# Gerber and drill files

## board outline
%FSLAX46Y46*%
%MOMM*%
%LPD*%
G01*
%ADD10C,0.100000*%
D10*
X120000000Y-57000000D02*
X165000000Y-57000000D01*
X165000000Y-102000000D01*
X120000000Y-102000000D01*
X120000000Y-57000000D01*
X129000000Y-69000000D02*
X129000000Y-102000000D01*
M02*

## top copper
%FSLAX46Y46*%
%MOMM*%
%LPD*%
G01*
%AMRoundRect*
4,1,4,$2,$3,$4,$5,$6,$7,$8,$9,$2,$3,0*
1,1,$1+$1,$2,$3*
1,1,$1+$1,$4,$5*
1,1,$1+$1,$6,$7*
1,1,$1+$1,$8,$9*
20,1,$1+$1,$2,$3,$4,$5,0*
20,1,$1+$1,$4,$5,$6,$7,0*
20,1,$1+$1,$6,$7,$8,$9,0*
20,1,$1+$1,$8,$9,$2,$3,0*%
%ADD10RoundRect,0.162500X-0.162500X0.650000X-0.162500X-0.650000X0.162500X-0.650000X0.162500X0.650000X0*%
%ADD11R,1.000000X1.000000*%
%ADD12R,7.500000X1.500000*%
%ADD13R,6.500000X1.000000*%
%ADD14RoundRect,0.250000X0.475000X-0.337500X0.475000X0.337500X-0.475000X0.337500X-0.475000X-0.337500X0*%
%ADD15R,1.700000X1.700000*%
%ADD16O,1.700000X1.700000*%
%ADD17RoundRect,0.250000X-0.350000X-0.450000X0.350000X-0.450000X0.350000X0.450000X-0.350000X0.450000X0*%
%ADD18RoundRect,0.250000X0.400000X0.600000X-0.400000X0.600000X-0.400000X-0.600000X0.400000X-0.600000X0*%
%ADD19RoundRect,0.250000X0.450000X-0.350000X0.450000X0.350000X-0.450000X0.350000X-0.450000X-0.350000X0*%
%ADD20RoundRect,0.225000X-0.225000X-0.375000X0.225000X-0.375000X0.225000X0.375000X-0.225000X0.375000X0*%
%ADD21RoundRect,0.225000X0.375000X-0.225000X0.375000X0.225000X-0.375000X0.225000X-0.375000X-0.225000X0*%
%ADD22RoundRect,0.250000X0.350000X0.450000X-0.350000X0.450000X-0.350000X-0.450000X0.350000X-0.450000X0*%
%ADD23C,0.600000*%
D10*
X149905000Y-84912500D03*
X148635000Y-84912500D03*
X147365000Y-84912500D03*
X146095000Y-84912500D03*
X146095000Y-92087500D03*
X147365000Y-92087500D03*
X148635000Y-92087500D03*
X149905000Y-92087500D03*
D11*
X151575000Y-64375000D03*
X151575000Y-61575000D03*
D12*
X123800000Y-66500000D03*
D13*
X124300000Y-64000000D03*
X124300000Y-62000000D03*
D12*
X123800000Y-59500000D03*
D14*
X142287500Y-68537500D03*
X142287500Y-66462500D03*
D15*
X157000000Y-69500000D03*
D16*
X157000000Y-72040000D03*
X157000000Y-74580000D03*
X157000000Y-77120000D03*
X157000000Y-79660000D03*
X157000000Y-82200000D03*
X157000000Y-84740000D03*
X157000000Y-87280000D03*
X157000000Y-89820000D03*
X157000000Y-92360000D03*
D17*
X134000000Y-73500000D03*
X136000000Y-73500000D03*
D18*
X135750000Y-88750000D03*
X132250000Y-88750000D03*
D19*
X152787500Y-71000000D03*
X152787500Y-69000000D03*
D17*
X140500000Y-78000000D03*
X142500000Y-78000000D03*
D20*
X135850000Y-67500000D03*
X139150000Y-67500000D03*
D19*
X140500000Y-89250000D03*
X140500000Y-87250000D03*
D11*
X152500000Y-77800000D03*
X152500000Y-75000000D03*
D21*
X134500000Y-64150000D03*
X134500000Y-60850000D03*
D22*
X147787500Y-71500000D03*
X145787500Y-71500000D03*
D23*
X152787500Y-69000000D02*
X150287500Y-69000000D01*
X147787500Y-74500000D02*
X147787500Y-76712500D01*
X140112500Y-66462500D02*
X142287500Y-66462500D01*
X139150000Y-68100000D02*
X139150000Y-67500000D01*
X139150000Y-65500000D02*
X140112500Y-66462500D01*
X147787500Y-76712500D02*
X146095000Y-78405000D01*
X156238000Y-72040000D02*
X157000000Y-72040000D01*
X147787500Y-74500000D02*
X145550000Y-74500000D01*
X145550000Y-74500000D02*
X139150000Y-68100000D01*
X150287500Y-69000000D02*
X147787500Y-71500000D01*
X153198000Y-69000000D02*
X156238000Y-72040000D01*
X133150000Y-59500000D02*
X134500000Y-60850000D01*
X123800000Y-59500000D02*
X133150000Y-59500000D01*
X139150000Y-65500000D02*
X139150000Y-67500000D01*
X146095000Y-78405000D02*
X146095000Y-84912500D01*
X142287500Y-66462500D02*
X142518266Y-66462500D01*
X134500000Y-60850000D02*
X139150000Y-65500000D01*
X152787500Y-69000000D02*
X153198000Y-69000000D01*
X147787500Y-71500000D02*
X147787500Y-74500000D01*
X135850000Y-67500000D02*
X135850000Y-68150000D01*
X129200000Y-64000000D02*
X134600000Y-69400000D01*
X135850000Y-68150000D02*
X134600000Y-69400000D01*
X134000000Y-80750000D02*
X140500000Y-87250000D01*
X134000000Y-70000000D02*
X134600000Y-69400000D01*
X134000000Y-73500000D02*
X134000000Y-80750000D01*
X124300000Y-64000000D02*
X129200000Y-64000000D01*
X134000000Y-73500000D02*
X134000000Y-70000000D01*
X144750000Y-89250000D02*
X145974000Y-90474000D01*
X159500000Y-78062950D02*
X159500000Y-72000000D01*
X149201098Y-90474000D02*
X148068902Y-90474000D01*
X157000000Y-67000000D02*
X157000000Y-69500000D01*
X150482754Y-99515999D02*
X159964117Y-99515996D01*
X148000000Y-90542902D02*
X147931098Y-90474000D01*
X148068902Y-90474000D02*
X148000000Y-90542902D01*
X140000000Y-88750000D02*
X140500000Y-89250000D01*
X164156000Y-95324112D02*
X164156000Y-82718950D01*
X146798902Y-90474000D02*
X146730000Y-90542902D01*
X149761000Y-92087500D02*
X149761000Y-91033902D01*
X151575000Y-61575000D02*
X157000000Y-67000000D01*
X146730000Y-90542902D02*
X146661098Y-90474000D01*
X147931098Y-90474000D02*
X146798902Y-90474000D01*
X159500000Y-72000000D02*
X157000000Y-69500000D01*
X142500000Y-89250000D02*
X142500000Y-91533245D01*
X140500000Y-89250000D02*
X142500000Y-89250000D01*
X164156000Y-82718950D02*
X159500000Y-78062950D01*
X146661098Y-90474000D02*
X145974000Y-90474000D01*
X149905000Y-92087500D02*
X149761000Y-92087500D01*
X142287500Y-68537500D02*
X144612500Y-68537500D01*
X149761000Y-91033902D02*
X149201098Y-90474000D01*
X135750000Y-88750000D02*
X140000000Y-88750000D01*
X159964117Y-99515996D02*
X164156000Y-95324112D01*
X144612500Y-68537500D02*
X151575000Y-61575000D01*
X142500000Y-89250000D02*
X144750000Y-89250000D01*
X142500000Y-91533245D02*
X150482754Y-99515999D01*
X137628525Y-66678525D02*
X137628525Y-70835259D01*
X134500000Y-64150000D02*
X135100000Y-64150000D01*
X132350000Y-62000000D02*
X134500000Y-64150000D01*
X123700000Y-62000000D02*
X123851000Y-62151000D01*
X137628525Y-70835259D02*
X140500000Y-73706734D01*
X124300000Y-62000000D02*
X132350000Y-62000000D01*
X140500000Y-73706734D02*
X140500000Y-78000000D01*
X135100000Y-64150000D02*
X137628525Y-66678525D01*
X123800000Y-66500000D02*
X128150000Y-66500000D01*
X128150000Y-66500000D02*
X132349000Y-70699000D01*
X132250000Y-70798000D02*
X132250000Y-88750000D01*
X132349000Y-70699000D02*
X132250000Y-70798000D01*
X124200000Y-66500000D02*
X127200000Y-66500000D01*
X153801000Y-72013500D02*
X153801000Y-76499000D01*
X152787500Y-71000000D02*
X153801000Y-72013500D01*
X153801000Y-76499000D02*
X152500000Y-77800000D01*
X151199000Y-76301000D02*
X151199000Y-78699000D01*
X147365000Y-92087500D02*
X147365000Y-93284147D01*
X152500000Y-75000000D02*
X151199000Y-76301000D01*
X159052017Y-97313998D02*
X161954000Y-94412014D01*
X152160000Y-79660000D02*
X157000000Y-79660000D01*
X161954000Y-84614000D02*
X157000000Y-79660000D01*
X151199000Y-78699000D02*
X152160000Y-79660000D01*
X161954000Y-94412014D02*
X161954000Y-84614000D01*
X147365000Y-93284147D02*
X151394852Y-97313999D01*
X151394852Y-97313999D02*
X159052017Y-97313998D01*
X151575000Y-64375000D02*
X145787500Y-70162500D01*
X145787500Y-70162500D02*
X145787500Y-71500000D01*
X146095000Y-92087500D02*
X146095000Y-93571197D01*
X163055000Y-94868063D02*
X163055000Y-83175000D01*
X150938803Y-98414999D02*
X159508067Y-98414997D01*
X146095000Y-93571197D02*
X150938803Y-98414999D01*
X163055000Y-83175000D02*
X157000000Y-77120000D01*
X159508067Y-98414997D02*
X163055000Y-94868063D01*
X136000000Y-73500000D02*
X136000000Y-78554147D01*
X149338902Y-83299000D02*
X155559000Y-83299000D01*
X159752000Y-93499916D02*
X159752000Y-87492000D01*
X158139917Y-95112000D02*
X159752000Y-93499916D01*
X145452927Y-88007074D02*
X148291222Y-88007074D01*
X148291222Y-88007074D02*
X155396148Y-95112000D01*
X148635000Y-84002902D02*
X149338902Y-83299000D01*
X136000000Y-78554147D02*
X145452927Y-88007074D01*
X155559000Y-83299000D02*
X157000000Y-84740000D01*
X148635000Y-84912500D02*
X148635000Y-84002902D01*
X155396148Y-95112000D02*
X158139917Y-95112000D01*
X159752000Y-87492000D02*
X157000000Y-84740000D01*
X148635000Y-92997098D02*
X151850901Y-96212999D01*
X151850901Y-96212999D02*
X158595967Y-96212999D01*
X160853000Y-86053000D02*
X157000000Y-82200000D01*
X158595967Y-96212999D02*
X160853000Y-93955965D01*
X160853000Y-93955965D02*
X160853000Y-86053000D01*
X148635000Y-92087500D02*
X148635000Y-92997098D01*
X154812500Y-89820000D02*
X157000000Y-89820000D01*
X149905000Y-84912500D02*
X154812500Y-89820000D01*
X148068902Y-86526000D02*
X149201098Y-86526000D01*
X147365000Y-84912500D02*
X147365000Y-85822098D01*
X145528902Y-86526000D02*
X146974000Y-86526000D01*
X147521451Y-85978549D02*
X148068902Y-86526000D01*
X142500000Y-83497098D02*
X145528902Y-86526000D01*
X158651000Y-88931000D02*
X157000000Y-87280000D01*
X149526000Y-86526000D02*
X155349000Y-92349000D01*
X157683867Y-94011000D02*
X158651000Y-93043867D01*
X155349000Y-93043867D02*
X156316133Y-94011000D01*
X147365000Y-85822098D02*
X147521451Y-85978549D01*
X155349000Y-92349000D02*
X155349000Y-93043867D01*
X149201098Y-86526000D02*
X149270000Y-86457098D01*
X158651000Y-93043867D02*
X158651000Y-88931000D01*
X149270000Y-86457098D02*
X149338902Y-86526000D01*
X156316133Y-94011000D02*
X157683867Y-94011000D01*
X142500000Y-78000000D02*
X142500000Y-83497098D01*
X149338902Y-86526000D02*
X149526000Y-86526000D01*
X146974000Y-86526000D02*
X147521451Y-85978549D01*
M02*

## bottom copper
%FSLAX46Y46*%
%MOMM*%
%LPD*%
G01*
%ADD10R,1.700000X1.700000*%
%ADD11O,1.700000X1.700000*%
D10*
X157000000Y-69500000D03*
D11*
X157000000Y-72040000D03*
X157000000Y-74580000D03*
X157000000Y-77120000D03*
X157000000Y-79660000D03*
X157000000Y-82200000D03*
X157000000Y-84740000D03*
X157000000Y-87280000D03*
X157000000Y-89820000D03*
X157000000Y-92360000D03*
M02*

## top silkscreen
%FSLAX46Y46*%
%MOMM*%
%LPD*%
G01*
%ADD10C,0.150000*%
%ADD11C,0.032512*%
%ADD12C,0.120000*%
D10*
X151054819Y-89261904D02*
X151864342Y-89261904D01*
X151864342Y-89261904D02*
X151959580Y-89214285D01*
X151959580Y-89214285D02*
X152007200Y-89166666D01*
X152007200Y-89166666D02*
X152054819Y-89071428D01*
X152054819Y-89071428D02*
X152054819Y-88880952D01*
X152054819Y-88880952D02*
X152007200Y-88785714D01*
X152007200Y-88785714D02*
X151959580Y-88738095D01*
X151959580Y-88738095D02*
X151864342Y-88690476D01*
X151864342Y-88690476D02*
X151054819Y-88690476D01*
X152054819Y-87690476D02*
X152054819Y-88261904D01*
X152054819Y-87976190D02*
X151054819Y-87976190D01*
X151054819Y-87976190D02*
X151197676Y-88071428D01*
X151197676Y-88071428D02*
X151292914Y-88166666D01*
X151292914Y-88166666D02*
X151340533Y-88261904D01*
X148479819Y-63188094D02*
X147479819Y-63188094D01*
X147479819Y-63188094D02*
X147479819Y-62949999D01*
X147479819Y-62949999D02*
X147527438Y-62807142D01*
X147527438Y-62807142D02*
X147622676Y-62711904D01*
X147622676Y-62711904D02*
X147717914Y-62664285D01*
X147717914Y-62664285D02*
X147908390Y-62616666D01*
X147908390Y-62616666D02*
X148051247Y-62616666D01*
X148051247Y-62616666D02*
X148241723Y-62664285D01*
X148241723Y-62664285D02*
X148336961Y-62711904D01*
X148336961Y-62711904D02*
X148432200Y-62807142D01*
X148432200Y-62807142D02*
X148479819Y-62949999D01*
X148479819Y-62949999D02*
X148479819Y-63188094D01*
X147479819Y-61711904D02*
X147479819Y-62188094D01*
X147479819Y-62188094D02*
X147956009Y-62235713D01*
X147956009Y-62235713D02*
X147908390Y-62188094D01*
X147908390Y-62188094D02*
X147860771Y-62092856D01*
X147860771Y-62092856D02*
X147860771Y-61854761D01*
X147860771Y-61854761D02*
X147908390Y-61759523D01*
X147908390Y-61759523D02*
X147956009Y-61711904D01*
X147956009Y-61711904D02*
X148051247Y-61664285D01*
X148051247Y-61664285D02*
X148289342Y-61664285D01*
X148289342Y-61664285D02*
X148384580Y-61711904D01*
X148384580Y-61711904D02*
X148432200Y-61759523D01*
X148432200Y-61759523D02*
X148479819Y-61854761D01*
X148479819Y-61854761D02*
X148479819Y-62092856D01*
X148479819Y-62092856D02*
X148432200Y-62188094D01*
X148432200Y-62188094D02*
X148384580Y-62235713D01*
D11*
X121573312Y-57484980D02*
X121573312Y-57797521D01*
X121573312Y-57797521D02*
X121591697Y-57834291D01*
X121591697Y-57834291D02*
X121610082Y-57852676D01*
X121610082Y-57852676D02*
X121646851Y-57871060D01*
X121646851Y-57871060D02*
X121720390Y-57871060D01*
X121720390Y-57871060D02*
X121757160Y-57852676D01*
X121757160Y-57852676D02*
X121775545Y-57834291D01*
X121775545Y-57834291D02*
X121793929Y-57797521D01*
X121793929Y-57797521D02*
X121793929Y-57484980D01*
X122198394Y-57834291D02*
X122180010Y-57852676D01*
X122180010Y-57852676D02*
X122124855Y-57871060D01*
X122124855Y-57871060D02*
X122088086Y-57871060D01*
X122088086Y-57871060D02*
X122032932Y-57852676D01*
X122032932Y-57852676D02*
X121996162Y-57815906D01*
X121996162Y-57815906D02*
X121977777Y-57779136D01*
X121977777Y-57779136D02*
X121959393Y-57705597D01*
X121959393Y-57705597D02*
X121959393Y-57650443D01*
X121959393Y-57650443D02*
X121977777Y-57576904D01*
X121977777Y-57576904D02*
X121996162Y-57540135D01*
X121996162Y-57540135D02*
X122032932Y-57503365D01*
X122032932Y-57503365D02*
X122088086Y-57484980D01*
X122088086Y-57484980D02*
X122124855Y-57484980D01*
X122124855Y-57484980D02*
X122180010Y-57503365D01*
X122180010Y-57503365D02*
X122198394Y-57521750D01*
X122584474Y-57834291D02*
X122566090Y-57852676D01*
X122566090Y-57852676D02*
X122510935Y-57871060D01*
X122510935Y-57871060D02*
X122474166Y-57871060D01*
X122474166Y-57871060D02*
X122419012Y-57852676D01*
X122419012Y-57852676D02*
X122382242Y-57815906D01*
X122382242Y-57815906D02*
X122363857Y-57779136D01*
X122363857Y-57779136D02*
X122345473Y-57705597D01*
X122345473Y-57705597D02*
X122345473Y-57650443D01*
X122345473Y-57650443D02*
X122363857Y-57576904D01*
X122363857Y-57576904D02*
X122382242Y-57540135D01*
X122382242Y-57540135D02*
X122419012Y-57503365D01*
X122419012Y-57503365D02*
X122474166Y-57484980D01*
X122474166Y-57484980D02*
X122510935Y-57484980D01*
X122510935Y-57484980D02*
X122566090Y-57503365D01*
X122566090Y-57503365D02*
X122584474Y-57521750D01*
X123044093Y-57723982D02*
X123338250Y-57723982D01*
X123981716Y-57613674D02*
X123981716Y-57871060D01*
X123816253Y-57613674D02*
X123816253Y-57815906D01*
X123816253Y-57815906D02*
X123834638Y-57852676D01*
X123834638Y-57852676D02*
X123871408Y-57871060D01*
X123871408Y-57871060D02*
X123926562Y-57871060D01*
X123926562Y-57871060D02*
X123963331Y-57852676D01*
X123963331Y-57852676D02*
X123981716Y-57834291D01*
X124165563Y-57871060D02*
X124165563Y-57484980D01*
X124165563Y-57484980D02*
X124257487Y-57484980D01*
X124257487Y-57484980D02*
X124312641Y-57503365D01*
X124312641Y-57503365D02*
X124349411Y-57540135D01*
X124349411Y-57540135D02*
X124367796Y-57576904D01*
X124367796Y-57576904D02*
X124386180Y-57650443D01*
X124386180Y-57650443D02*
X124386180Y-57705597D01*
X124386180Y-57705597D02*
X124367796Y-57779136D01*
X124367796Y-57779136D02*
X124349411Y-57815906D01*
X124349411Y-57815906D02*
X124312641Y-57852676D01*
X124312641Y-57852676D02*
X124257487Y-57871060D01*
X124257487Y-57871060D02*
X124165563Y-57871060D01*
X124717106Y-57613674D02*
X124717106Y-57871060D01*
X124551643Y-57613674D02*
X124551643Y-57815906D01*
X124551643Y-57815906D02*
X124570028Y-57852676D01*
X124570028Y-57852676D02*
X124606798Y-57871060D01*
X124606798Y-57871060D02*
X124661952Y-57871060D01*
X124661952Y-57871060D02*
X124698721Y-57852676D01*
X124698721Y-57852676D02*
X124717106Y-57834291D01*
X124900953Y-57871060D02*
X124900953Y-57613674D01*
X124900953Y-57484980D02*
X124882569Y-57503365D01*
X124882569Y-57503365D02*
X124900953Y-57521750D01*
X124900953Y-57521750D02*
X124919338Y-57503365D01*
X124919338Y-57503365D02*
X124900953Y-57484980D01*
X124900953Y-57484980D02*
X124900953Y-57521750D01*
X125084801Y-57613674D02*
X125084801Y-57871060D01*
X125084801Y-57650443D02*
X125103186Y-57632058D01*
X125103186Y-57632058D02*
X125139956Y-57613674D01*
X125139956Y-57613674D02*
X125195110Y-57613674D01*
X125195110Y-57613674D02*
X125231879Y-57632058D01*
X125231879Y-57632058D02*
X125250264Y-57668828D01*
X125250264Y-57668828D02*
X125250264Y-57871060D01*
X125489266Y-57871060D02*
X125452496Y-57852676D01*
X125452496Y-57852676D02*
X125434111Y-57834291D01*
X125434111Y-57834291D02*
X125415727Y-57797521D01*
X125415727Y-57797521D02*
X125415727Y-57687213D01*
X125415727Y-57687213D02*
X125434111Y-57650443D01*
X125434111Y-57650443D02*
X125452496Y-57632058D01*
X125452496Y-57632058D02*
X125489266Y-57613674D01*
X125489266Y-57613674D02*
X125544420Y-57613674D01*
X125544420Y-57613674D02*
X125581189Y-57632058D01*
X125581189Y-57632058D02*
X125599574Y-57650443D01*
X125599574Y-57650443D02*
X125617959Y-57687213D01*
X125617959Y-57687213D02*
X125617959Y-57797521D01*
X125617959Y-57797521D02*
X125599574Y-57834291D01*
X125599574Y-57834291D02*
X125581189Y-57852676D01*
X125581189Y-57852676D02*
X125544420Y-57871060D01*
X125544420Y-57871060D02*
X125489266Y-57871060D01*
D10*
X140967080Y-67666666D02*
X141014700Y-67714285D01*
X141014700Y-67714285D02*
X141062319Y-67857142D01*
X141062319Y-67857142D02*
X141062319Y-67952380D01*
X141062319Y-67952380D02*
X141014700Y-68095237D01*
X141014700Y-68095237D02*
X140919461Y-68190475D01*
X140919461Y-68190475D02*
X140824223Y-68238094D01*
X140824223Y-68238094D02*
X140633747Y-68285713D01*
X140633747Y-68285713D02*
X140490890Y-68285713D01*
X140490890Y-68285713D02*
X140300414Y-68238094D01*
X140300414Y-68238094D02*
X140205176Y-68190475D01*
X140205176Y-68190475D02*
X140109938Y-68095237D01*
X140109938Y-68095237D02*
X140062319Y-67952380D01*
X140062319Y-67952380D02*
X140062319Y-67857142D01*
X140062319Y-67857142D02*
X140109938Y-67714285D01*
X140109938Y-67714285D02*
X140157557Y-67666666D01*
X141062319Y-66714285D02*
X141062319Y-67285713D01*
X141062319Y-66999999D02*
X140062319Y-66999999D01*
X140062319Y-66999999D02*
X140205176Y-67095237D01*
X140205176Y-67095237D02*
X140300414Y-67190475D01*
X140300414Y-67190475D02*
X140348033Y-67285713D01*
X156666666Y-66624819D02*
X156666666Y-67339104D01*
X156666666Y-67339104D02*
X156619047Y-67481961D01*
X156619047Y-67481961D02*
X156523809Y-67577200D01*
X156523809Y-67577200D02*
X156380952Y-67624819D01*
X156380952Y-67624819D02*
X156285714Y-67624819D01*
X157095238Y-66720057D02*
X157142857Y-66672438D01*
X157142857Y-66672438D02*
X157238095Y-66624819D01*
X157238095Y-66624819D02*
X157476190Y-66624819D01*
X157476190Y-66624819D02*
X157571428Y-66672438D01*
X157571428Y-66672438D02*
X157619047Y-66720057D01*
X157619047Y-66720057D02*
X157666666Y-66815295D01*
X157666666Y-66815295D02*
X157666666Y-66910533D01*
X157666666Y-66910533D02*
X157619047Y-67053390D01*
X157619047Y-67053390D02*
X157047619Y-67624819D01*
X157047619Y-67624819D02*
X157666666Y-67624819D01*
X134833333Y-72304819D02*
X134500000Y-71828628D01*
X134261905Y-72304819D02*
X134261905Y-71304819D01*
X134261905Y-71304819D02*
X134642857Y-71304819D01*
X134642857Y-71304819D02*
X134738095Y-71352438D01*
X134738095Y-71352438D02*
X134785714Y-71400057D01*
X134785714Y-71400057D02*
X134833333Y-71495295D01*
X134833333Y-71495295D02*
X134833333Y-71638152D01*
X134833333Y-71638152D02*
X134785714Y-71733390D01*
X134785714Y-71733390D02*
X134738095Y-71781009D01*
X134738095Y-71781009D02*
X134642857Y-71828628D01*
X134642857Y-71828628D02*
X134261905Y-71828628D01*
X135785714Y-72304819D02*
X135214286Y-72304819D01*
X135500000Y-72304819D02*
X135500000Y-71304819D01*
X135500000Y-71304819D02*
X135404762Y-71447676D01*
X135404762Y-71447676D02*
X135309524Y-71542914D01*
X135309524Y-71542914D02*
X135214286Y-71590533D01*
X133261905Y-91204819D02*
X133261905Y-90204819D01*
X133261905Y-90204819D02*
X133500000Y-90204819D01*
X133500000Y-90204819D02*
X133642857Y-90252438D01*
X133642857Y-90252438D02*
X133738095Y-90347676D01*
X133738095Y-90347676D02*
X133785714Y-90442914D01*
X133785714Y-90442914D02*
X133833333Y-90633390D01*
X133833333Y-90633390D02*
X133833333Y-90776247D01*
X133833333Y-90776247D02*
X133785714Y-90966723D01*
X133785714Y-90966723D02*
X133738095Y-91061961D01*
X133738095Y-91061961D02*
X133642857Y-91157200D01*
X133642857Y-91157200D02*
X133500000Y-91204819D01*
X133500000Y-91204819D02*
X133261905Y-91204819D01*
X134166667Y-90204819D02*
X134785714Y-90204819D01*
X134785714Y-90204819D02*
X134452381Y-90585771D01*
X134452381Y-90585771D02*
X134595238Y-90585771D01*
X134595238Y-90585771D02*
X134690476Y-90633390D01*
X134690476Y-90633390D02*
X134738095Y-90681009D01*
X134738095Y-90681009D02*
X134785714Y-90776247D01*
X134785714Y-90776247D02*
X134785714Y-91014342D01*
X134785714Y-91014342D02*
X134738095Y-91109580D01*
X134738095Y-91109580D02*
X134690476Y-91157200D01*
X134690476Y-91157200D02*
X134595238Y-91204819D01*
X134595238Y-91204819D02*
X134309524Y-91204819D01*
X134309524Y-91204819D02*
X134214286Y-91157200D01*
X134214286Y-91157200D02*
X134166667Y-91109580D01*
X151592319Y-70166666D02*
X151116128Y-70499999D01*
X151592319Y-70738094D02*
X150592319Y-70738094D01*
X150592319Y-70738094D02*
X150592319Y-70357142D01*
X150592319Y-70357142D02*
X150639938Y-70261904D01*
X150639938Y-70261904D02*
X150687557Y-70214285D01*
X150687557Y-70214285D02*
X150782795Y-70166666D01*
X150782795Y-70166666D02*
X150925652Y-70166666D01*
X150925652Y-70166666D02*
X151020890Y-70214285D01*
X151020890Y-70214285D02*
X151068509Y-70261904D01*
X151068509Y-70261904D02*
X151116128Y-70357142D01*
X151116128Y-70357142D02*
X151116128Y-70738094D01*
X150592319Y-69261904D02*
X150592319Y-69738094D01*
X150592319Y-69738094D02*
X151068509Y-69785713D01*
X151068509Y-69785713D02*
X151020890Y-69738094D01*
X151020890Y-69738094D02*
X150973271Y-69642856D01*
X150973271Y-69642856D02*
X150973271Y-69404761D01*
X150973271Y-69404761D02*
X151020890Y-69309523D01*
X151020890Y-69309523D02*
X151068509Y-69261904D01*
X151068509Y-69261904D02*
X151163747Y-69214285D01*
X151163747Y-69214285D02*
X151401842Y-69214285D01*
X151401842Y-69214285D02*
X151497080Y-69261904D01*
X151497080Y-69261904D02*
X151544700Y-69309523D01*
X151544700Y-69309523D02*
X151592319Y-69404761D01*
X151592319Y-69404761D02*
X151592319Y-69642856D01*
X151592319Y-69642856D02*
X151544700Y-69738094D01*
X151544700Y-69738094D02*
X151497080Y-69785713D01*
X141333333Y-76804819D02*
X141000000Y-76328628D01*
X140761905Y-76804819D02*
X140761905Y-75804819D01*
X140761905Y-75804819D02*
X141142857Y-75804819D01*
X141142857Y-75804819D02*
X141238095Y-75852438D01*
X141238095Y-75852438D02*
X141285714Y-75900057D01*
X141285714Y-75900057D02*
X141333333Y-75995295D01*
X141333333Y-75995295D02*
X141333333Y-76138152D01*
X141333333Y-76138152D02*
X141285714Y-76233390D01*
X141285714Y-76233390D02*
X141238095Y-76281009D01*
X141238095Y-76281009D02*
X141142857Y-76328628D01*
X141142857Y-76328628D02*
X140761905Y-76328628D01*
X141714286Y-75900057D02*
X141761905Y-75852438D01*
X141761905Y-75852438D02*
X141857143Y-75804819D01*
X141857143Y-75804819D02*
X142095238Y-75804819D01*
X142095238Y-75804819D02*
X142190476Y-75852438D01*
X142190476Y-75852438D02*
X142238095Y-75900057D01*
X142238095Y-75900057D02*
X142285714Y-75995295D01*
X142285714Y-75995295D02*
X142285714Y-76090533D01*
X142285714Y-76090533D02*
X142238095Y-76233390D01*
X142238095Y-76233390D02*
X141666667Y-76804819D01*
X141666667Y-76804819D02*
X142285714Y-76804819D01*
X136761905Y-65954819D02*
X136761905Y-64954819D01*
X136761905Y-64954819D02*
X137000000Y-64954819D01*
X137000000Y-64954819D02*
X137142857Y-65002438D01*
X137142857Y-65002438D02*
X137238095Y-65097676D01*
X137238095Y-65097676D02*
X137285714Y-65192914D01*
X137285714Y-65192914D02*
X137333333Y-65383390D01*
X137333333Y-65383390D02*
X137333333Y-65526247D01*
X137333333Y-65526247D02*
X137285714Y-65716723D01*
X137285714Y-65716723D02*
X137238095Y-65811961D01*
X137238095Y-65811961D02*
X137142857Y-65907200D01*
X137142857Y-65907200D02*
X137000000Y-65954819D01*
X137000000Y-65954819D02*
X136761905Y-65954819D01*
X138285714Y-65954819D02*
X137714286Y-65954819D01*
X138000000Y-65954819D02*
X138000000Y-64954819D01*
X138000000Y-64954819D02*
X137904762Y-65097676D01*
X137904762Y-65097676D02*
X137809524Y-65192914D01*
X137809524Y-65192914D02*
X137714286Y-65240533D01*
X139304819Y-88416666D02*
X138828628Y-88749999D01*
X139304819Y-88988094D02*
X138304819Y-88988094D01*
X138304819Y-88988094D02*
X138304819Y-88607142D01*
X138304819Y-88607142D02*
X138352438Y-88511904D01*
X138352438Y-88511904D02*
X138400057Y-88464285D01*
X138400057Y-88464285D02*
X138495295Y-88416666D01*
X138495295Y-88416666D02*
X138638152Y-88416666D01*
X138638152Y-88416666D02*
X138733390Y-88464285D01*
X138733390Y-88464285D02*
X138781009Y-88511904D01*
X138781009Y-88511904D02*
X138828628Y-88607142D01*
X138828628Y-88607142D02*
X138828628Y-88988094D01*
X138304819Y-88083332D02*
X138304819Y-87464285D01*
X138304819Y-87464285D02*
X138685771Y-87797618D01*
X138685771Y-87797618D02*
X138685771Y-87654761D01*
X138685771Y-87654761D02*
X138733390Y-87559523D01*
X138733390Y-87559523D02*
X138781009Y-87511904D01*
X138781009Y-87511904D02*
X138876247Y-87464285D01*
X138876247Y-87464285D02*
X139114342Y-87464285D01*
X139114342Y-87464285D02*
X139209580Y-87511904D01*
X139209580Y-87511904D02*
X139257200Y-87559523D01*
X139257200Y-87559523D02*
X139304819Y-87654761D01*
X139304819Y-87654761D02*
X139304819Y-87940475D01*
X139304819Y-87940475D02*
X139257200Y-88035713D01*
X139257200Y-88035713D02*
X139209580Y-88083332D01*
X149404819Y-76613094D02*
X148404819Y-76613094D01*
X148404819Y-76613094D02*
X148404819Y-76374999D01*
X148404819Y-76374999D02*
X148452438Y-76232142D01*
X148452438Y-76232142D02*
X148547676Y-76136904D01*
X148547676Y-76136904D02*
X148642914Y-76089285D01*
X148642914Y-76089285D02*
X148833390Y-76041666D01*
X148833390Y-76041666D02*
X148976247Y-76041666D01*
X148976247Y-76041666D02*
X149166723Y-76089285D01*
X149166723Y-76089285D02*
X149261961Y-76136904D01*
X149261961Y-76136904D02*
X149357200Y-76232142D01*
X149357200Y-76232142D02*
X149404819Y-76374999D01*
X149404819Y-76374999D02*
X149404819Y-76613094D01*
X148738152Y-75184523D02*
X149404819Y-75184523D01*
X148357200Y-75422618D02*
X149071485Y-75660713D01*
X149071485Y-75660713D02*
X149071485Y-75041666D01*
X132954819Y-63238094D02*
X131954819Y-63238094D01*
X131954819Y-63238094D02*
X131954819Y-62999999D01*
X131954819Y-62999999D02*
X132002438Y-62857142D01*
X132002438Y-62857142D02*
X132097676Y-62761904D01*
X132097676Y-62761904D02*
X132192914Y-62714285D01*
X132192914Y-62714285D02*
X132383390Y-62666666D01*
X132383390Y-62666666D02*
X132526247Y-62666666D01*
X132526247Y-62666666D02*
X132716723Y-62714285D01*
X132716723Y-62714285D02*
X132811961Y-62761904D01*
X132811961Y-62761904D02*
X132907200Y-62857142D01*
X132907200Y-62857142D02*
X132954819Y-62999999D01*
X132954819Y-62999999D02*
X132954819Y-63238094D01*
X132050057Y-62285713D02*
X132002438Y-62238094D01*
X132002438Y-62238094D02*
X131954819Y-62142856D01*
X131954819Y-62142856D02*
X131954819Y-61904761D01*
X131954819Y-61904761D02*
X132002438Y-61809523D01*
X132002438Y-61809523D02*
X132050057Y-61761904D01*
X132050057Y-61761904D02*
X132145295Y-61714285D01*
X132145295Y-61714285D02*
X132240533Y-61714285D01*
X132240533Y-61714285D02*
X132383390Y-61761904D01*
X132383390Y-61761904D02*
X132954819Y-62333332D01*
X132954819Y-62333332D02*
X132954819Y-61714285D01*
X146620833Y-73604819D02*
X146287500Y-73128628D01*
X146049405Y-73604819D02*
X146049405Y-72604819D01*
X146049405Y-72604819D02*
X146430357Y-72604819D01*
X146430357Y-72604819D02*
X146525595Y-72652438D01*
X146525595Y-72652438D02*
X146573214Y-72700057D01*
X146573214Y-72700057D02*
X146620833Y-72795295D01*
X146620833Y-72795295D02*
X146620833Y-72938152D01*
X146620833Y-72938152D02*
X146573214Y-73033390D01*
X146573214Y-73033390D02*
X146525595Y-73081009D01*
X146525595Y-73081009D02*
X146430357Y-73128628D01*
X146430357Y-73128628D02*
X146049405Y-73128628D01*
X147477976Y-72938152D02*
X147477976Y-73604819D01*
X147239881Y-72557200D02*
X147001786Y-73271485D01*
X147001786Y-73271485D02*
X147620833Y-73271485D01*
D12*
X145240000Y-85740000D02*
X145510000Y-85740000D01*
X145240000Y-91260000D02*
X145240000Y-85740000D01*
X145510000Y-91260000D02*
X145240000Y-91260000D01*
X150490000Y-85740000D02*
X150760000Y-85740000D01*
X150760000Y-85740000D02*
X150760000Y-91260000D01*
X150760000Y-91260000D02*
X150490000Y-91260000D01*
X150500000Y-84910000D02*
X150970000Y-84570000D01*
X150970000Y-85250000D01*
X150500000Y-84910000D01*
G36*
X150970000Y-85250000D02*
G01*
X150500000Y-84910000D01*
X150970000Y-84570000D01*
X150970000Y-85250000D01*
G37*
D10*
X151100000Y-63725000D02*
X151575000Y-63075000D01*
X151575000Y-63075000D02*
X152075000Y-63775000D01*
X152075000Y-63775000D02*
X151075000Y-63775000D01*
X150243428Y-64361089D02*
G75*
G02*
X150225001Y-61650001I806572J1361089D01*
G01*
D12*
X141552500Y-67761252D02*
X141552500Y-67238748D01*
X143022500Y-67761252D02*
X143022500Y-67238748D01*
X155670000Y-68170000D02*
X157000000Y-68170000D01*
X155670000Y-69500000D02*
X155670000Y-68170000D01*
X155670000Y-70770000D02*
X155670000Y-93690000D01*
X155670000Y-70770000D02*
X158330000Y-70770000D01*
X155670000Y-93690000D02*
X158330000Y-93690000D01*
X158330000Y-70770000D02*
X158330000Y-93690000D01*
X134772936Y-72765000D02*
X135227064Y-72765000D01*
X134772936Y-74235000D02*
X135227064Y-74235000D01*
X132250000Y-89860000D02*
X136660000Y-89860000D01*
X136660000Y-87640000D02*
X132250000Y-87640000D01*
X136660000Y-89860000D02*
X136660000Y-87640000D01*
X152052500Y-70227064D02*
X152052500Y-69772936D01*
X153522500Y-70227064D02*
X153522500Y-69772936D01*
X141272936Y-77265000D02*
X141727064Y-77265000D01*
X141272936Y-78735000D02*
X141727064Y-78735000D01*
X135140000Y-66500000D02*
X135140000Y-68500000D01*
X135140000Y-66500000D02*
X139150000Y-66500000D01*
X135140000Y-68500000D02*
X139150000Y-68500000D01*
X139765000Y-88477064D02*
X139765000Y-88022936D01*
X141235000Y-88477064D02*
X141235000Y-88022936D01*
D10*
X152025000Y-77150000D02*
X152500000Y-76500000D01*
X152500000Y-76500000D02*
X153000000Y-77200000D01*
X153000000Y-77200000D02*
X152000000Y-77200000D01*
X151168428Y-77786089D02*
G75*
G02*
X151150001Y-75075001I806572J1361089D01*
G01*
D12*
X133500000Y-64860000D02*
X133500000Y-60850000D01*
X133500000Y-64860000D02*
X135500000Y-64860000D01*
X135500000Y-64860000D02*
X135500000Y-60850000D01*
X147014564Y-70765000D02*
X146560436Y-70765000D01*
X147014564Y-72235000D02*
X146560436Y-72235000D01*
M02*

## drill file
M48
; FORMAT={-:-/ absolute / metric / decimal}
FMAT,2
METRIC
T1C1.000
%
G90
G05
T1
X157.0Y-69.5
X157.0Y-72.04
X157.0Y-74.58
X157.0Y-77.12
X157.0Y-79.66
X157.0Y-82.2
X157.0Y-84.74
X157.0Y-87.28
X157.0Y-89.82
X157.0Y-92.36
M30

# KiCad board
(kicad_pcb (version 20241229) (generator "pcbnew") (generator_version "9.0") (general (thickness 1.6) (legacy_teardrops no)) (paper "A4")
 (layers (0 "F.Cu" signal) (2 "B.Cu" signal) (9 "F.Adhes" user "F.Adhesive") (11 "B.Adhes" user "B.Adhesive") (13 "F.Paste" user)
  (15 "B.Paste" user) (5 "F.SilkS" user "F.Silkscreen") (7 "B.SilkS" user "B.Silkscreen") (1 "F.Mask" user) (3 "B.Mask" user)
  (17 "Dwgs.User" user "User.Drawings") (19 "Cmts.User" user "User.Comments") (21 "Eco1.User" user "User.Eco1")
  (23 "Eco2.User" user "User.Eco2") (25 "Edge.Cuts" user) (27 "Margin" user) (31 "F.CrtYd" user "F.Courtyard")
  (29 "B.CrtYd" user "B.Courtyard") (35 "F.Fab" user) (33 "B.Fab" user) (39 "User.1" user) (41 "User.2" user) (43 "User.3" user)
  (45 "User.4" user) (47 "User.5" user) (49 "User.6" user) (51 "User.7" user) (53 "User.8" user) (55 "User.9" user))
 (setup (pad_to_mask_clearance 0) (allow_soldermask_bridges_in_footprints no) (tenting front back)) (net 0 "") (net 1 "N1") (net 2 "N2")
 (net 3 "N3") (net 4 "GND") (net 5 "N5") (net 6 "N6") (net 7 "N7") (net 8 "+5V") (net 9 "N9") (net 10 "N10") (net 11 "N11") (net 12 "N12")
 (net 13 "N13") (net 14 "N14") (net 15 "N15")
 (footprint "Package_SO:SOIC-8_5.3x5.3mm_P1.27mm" (layer "F.Cu") (at 148 88.5 -90)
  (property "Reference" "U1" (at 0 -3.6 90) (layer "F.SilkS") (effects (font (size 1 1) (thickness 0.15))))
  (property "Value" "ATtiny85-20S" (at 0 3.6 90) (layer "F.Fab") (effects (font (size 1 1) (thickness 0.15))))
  (fp_line (start -2.76 2.76) (end -2.76 2.49) (stroke (width 0.12) (type solid)) (layer "F.SilkS"))
  (fp_line (start 2.76 2.76) (end -2.76 2.76) (stroke (width 0.12) (type solid)) (layer "F.SilkS"))
  (fp_line (start 2.76 2.49) (end 2.76 2.76) (stroke (width 0.12) (type solid)) (layer "F.SilkS"))
  (fp_line (start -2.76 -2.49) (end -2.76 -2.76) (stroke (width 0.12) (type solid)) (layer "F.SilkS"))
  (fp_line (start -2.76 -2.76) (end 2.76 -2.76) (stroke (width 0.12) (type solid)) (layer "F.SilkS"))
  (fp_line (start 2.76 -2.76) (end 2.76 -2.49) (stroke (width 0.12) (type solid)) (layer "F.SilkS"))
  (fp_poly (pts (xy -3.59 -2.5) (xy -3.93 -2.97) (xy -3.25 -2.97)) (stroke (width 0.12) (type solid)) (fill yes) (layer "F.SilkS"))
  (pad "1" smd roundrect (at -3.5875 -1.905 270) (size 1.625 0.65) (layers "F.Cu" "F.Mask" "F.Paste") (roundrect_rratio 0.25) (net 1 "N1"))
  (pad "2" smd roundrect (at -3.5875 -0.635 270) (size 1.625 0.65) (layers "F.Cu" "F.Mask" "F.Paste") (roundrect_rratio 0.25) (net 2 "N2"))
  (pad "3" smd roundrect (at -3.5875 0.635 270) (size 1.625 0.65) (layers "F.Cu" "F.Mask" "F.Paste") (roundrect_rratio 0.25) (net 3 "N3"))
  (pad "4" smd roundrect (at -3.5875 1.905 270) (size 1.625 0.65) (layers "F.Cu" "F.Mask" "F.Paste") (roundrect_rratio 0.25) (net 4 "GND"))
  (pad "5" smd roundrect (at 3.5875 1.905 270) (size 1.625 0.65) (layers "F.Cu" "F.Mask" "F.Paste") (roundrect_rratio 0.25) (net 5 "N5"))
  (pad "6" smd roundrect (at 3.5875 0.635 270) (size 1.625 0.65) (layers "F.Cu" "F.Mask" "F.Paste") (roundrect_rratio 0.25) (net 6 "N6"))
  (pad "7" smd roundrect (at 3.5875 -0.635 270) (size 1.625 0.65) (layers "F.Cu" "F.Mask" "F.Paste") (roundrect_rratio 0.25) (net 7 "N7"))
  (pad "8" smd roundrect (at 3.5875 -1.905 270) (size 1.625 0.65) (layers "F.Cu" "F.Mask" "F.Paste") (roundrect_rratio 0.25) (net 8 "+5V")))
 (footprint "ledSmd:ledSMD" (layer "F.Cu") (at 151.575 62.575 90)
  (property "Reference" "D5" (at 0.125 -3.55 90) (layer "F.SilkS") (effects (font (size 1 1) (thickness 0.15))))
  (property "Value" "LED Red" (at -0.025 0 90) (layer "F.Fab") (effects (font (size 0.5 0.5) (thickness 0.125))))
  (fp_line (start -1.15 -0.475) (end -0.5 0) (stroke (width 0.15) (type solid)) (layer "F.SilkS"))
  (fp_line (start -0.5 0) (end -1.2 0.5) (stroke (width 0.15) (type solid)) (layer "F.SilkS"))
  (fp_line (start -1.2 0.5) (end -1.2 -0.5) (stroke (width 0.15) (type solid)) (layer "F.SilkS"))
  (fp_arc (start -1.786089 -1.331572) (mid -0.435753 -2.107089) (end 0.924999 -1.349999) (stroke (width 0.15) (type solid))
   (layer "F.SilkS"))
  (pad "1" smd rect (at -1.8 0 90) (size 1 1) (layers "F.Cu" "F.Mask" "F.Paste") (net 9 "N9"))
  (pad "2" smd rect (at 1 0 90) (size 1 1) (layers "F.Cu" "F.Mask" "F.Paste") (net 8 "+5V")))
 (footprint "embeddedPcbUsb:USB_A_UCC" (layer "F.Cu") (at 124 63)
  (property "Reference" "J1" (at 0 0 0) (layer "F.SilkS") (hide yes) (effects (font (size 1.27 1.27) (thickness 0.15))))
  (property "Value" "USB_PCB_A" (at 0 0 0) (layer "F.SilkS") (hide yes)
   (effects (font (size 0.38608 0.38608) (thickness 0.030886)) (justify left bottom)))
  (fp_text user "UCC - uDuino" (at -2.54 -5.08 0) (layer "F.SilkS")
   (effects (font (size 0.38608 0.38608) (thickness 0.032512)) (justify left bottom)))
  (pad "1" smd rect (at -0.2 3.5) (size 7.5 1.5) (layers "F.Cu" "F.Mask" "F.Paste") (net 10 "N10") (solder_mask_margin 0.1016))
  (pad "2" smd rect (at 0.3 1) (size 6.5 1) (layers "F.Cu" "F.Mask" "F.Paste") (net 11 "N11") (solder_mask_margin 0.1016))
  (pad "3" smd rect (at 0.3 -1) (size 6.5 1) (layers "F.Cu" "F.Mask" "F.Paste") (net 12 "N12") (solder_mask_margin 0.1016))
  (pad "4" smd rect (at -0.2 -3.5) (size 7.5 1.5) (layers "F.Cu" "F.Mask" "F.Paste") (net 4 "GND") (solder_mask_margin 0.1016)))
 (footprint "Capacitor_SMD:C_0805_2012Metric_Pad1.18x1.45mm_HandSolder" (layer "F.Cu") (at 142.2875 67.5 90)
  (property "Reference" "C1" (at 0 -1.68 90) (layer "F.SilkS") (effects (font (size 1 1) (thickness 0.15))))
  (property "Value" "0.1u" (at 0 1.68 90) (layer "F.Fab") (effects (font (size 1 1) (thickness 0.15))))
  (fp_line (start -0.261252 -0.735) (end 0.261252 -0.735) (stroke (width 0.12) (type solid)) (layer "F.SilkS"))
  (fp_line (start -0.261252 0.735) (end 0.261252 0.735) (stroke (width 0.12) (type solid)) (layer "F.SilkS"))
  (pad "1" smd roundrect (at -1.0375 0 90) (size 1.175 1.45) (layers "F.Cu" "F.Mask" "F.Paste") (roundrect_rratio 0.212766) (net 8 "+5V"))
  (pad "2" smd roundrect (at 1.0375 0 90) (size 1.175 1.45) (layers "F.Cu" "F.Mask" "F.Paste") (roundrect_rratio 0.212766) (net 4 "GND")))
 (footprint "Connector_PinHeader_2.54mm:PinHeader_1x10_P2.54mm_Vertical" (layer "F.Cu") (at 157 69.5)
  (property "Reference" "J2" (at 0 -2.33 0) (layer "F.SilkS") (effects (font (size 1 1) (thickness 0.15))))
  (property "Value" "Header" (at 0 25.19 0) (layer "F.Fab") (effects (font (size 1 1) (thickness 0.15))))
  (fp_line (start -1.33 -1.33) (end 0 -1.33) (stroke (width 0.12) (type solid)) (layer "F.SilkS"))
  (fp_line (start -1.33 0) (end -1.33 -1.33) (stroke (width 0.12) (type solid)) (layer "F.SilkS"))
  (fp_line (start -1.33 1.27) (end -1.33 24.19) (stroke (width 0.12) (type solid)) (layer "F.SilkS"))
  (fp_line (start -1.33 1.27) (end 1.33 1.27) (stroke (width 0.12) (type solid)) (layer "F.SilkS"))
  (fp_line (start -1.33 24.19) (end 1.33 24.19) (stroke (width 0.12) (type solid)) (layer "F.SilkS"))
  (fp_line (start 1.33 1.27) (end 1.33 24.19) (stroke (width 0.12) (type solid)) (layer "F.SilkS"))
  (pad "1" thru_hole rect (at 0 0) (size 1.7 1.7) (drill 1) (layers "*.Cu" "*.Mask") (remove_unused_layers no) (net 8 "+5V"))
  (pad "2" thru_hole oval (at 0 2.54) (size 1.7 1.7) (drill 1) (layers "*.Cu" "*.Mask") (remove_unused_layers no) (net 4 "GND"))
  (pad "3" thru_hole oval (at 0 5.08) (size 1.7 1.7) (drill 1) (layers "*.Cu" "*.Mask") (remove_unused_layers no) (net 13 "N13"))
  (pad "4" thru_hole oval (at 0 7.62) (size 1.7 1.7) (drill 1) (layers "*.Cu" "*.Mask") (remove_unused_layers no) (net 5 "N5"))
  (pad "5" thru_hole oval (at 0 10.16) (size 1.7 1.7) (drill 1) (layers "*.Cu" "*.Mask") (remove_unused_layers no) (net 6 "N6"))
  (pad "6" thru_hole oval (at 0 12.7) (size 1.7 1.7) (drill 1) (layers "*.Cu" "*.Mask") (remove_unused_layers no) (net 7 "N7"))
  (pad "7" thru_hole oval (at 0 15.24) (size 1.7 1.7) (drill 1) (layers "*.Cu" "*.Mask") (remove_unused_layers no) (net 2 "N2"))
  (pad "8" thru_hole oval (at 0 17.78) (size 1.7 1.7) (drill 1) (layers "*.Cu" "*.Mask") (remove_unused_layers no) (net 3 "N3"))
  (pad "9" thru_hole oval (at 0 20.32) (size 1.7 1.7) (drill 1) (layers "*.Cu" "*.Mask") (remove_unused_layers no) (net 1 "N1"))
  (pad "10" thru_hole oval (at 0 22.86) (size 1.7 1.7) (drill 1) (layers "*.Cu" "*.Mask") (remove_unused_layers no) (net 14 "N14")))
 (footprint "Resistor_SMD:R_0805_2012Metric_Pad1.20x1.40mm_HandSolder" (layer "F.Cu") (at 135 73.5)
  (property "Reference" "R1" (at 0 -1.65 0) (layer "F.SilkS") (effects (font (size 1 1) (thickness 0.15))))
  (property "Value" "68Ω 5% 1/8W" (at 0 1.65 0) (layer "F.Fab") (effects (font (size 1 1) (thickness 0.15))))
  (fp_line (start -0.227064 -0.735) (end 0.227064 -0.735) (stroke (width 0.12) (type solid)) (layer "F.SilkS"))
  (fp_line (start -0.227064 0.735) (end 0.227064 0.735) (stroke (width 0.12) (type solid)) (layer "F.SilkS"))
  (pad "1" smd roundrect (at -1 0) (size 1.2 1.4) (layers "F.Cu" "F.Mask" "F.Paste") (roundrect_rratio 0.208333) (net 11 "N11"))
  (pad "2" smd roundrect (at 1 0) (size 1.2 1.4) (layers "F.Cu" "F.Mask" "F.Paste") (roundrect_rratio 0.208333) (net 2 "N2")))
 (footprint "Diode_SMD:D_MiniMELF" (layer "F.Cu") (at 134 88.75 180)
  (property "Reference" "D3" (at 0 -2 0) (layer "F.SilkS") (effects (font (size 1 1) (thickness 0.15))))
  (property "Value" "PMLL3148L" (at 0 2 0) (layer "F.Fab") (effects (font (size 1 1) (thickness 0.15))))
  (fp_line (start 1.75 -1.11) (end -2.66 -1.11) (stroke (width 0.12) (type solid)) (layer "F.SilkS"))
  (fp_line (start -2.66 1.11) (end 1.75 1.11) (stroke (width 0.12) (type solid)) (layer "F.SilkS"))
  (fp_line (start -2.66 -1.11) (end -2.66 1.11) (stroke (width 0.12) (type solid)) (layer "F.SilkS"))
  (pad "1" smd roundrect (at -1.75 0 180) (size 1.3 1.7) (layers "F.Cu" "F.Mask" "F.Paste") (roundrect_rratio 0.1923076923) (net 8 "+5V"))
  (pad "2" smd roundrect (at 1.75 0 180) (size 1.3 1.7) (layers "F.Cu" "F.Mask" "F.Paste") (roundrect_rratio 0.1923076923) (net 10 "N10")))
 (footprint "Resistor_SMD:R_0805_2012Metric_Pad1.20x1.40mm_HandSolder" (layer "F.Cu") (at 152.7875 70 90)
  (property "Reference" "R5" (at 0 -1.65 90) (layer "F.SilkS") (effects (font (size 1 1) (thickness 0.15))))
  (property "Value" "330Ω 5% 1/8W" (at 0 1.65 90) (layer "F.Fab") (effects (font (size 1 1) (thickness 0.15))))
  (fp_line (start -0.227064 -0.735) (end 0.227064 -0.735) (stroke (width 0.12) (type solid)) (layer "F.SilkS"))
  (fp_line (start -0.227064 0.735) (end 0.227064 0.735) (stroke (width 0.12) (type solid)) (layer "F.SilkS"))
  (pad "1" smd roundrect (at -1 0 90) (size 1.2 1.4) (layers "F.Cu" "F.Mask" "F.Paste") (roundrect_rratio 0.208333) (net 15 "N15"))
  (pad "2" smd roundrect (at 1 0 90) (size 1.2 1.4) (layers "F.Cu" "F.Mask" "F.Paste") (roundrect_rratio 0.208333) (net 4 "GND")))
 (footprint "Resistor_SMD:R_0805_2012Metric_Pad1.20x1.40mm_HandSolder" (layer "F.Cu") (at 141.5 78)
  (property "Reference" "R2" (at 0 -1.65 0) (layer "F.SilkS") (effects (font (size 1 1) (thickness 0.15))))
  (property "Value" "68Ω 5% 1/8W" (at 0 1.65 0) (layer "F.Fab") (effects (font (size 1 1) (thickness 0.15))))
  (fp_line (start -0.227064 -0.735) (end 0.227064 -0.735) (stroke (width 0.12) (type solid)) (layer "F.SilkS"))
  (fp_line (start -0.227064 0.735) (end 0.227064 0.735) (stroke (width 0.12) (type solid)) (layer "F.SilkS"))
  (pad "1" smd roundrect (at -1 0) (size 1.2 1.4) (layers "F.Cu" "F.Mask" "F.Paste") (roundrect_rratio 0.208333) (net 12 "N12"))
  (pad "2" smd roundrect (at 1 0) (size 1.2 1.4) (layers "F.Cu" "F.Mask" "F.Paste") (roundrect_rratio 0.208333) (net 3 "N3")))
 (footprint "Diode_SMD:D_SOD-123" (layer "F.Cu") (at 137.5 67.5)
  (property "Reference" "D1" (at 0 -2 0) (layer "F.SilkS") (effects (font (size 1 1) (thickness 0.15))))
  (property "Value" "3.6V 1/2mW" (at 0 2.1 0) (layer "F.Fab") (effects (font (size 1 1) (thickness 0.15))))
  (fp_line (start -2.36 -1) (end -2.36 1) (stroke (width 0.12) (type solid)) (layer "F.SilkS"))
  (fp_line (start -2.36 -1) (end 1.65 -1) (stroke (width 0.12) (type solid)) (layer "F.SilkS"))
  (fp_line (start -2.36 1) (end 1.65 1) (stroke (width 0.12) (type solid)) (layer "F.SilkS"))
  (pad "1" smd roundrect (at -1.65 0) (size 0.9 1.2) (layers "F.Cu" "F.Mask" "F.Paste") (roundrect_rratio 0.25) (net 11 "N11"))
  (pad "2" smd roundrect (at 1.65 0) (size 0.9 1.2) (layers "F.Cu" "F.Mask" "F.Paste") (roundrect_rratio 0.25) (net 4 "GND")))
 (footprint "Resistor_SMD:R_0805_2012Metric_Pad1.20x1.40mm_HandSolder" (layer "F.Cu") (at 140.5 88.25 90)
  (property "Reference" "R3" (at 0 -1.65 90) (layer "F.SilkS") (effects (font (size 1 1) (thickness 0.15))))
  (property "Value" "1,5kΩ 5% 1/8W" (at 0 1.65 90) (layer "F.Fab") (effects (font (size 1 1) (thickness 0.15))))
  (fp_line (start -0.227064 -0.735) (end 0.227064 -0.735) (stroke (width 0.12) (type solid)) (layer "F.SilkS"))
  (fp_line (start -0.227064 0.735) (end 0.227064 0.735) (stroke (width 0.12) (type solid)) (layer "F.SilkS"))
  (pad "1" smd roundrect (at -1 0 90) (size 1.2 1.4) (layers "F.Cu" "F.Mask" "F.Paste") (roundrect_rratio 0.208333) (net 8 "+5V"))
  (pad "2" smd roundrect (at 1 0 90) (size 1.2 1.4) (layers "F.Cu" "F.Mask" "F.Paste") (roundrect_rratio 0.208333) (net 11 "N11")))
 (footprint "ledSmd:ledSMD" (layer "F.Cu") (at 152.5 76 90)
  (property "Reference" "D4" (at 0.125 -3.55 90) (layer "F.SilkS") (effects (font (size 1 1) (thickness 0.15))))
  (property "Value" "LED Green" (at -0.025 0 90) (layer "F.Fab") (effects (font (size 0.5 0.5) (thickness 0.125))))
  (fp_line (start -1.15 -0.475) (end -0.5 0) (stroke (width 0.15) (type solid)) (layer "F.SilkS"))
  (fp_line (start -0.5 0) (end -1.2 0.5) (stroke (width 0.15) (type solid)) (layer "F.SilkS"))
  (fp_line (start -1.2 0.5) (end -1.2 -0.5) (stroke (width 0.15) (type solid)) (layer "F.SilkS"))
  (fp_arc (start -1.786089 -1.331572) (mid -0.435753 -2.107089) (end 0.924999 -1.349999) (stroke (width 0.15) (type solid))
   (layer "F.SilkS"))
  (pad "1" smd rect (at -1.8 0 90) (size 1 1) (layers "F.Cu" "F.Mask" "F.Paste") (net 15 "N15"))
  (pad "2" smd rect (at 1 0 90) (size 1 1) (layers "F.Cu" "F.Mask" "F.Paste") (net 6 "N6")))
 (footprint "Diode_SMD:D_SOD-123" (layer "F.Cu") (at 134.5 62.5 90)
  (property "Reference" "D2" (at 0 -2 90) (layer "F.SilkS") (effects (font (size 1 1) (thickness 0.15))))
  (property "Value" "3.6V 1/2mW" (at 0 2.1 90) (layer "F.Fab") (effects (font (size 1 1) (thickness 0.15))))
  (fp_line (start -2.36 -1) (end 1.65 -1) (stroke (width 0.12) (type solid)) (layer "F.SilkS"))
  (fp_line (start -2.36 -1) (end -2.36 1) (stroke (width 0.12) (type solid)) (layer "F.SilkS"))
  (fp_line (start -2.36 1) (end 1.65 1) (stroke (width 0.12) (type solid)) (layer "F.SilkS"))
  (pad "1" smd roundrect (at -1.65 0 90) (size 0.9 1.2) (layers "F.Cu" "F.Mask" "F.Paste") (roundrect_rratio 0.25) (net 12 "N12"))
  (pad "2" smd roundrect (at 1.65 0 90) (size 0.9 1.2) (layers "F.Cu" "F.Mask" "F.Paste") (roundrect_rratio 0.25) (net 4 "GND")))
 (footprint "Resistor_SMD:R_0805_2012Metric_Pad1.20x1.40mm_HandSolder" (layer "F.Cu") (at 146.7875 71.5 180)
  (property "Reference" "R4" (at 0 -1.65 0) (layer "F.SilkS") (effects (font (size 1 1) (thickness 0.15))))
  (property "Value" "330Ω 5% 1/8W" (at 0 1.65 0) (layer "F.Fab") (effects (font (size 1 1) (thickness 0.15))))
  (fp_line (start -0.227064 0.735) (end 0.227064 0.735) (stroke (width 0.12) (type solid)) (layer "F.SilkS"))
  (fp_line (start -0.227064 -0.735) (end 0.227064 -0.735) (stroke (width 0.12) (type solid)) (layer "F.SilkS"))
  (pad "1" smd roundrect (at -1 0 180) (size 1.2 1.4) (layers "F.Cu" "F.Mask" "F.Paste") (roundrect_rratio 0.208333) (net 4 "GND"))
  (pad "2" smd roundrect (at 1 0 180) (size 1.2 1.4) (layers "F.Cu" "F.Mask" "F.Paste") (roundrect_rratio 0.208333) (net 9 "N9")))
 (gr_rect (start 120 57) (end 165 102) (stroke (width 0.1) (type default)) (fill no) (layer "Edge.Cuts"))
 (gr_line (start 129 69) (end 129 102) (stroke (width 0.1) (type default)) (layer "Edge.Cuts"))
 (segment (start 152.7875 69) (end 150.2875 69) (width 0.6) (layer "F.Cu") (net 4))
 (segment (start 147.7875 74.5) (end 147.7875 76.7125) (width 0.6) (layer "F.Cu") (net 4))
 (segment (start 140.1125 66.4625) (end 142.2875 66.4625) (width 0.6) (layer "F.Cu") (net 4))
 (segment (start 139.15 68.1) (end 139.15 67.5) (width 0.6) (layer "F.Cu") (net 4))
 (segment (start 139.15 65.5) (end 140.1125 66.4625) (width 0.6) (layer "F.Cu") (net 4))
 (segment (start 147.7875 76.7125) (end 146.095 78.405) (width 0.6) (layer "F.Cu") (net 4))
 (segment (start 156.238 72.04) (end 157 72.04) (width 0.6) (layer "F.Cu") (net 4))
 (segment (start 147.7875 74.5) (end 145.55 74.5) (width 0.6) (layer "F.Cu") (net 4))
 (segment (start 145.55 74.5) (end 139.15 68.1) (width 0.6) (layer "F.Cu") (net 4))
 (segment (start 150.2875 69) (end 147.7875 71.5) (width 0.6) (layer "F.Cu") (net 4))
 (segment (start 153.198 69) (end 156.238 72.04) (width 0.6) (layer "F.Cu") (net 4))
 (segment (start 133.15 59.5) (end 134.5 60.85) (width 0.6) (layer "F.Cu") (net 4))
 (segment (start 123.8 59.5) (end 133.15 59.5) (width 0.6) (layer "F.Cu") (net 4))
 (segment (start 139.15 65.5) (end 139.15 67.5) (width 0.6) (layer "F.Cu") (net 4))
 (segment (start 146.095 78.405) (end 146.095 84.9125) (width 0.6) (layer "F.Cu") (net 4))
 (segment (start 142.2875 66.4625) (end 142.518266 66.4625) (width 0.6) (layer "F.Cu") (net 4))
 (segment (start 134.5 60.85) (end 139.15 65.5) (width 0.6) (layer "F.Cu") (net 4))
 (segment (start 152.7875 69) (end 153.198 69) (width 0.6) (layer "F.Cu") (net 4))
 (segment (start 147.7875 71.5) (end 147.7875 74.5) (width 0.6) (layer "F.Cu") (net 4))
 (segment (start 135.85 67.5) (end 135.85 68.15) (width 0.6) (layer "F.Cu") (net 11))
 (segment (start 129.2 64) (end 134.6 69.4) (width 0.6) (layer "F.Cu") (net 11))
 (segment (start 135.85 68.15) (end 134.6 69.4) (width 0.6) (layer "F.Cu") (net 11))
 (segment (start 134 80.75) (end 140.5 87.25) (width 0.6) (layer "F.Cu") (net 11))
 (segment (start 134 70) (end 134.6 69.4) (width 0.6) (layer "F.Cu") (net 11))
 (segment (start 134 73.5) (end 134 80.75) (width 0.6) (layer "F.Cu") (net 11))
 (segment (start 124.3 64) (end 129.2 64) (width 0.6) (layer "F.Cu") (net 11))
 (segment (start 134 73.5) (end 134 70) (width 0.6) (layer "F.Cu") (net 11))
 (segment (start 144.75 89.25) (end 145.974 90.474) (width 0.6) (layer "F.Cu") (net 8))
 (segment (start 159.5 78.06295) (end 159.5 72) (width 0.6) (layer "F.Cu") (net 8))
 (segment (start 149.201098 90.474) (end 148.068902 90.474) (width 0.6) (layer "F.Cu") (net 8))
 (segment (start 157 67) (end 157 69.5) (width 0.6) (layer "F.Cu") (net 8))
 (segment (start 150.482754 99.515999) (end 159.964117 99.515996) (width 0.6) (layer "F.Cu") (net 8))
 (segment (start 148 90.542902) (end 147.931098 90.474) (width 0.6) (layer "F.Cu") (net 8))
 (segment (start 148.068902 90.474) (end 148 90.542902) (width 0.6) (layer "F.Cu") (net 8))
 (segment (start 140 88.75) (end 140.5 89.25) (width 0.6) (layer "F.Cu") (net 8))
 (segment (start 164.156 95.324112) (end 164.156 82.71895) (width 0.6) (layer "F.Cu") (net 8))
 (segment (start 146.798902 90.474) (end 146.73 90.542902) (width 0.6) (layer "F.Cu") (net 8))
 (segment (start 149.761 92.0875) (end 149.761 91.033902) (width 0.6) (layer "F.Cu") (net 8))
 (segment (start 151.575 61.575) (end 157 67) (width 0.6) (layer "F.Cu") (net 8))
 (segment (start 146.73 90.542902) (end 146.661098 90.474) (width 0.6) (layer "F.Cu") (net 8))
 (segment (start 147.931098 90.474) (end 146.798902 90.474) (width 0.6) (layer "F.Cu") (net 8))
 (segment (start 159.5 72) (end 157 69.5) (width 0.6) (layer "F.Cu") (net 8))
 (segment (start 142.5 89.25) (end 142.5 91.533245) (width 0.6) (layer "F.Cu") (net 8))
 (segment (start 140.5 89.25) (end 142.5 89.25) (width 0.6) (layer "F.Cu") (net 8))
 (segment (start 164.156 82.71895) (end 159.5 78.06295) (width 0.6) (layer "F.Cu") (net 8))
 (segment (start 146.661098 90.474) (end 145.974 90.474) (width 0.6) (layer "F.Cu") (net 8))
 (segment (start 149.905 92.0875) (end 149.761 92.0875) (width 0.6) (layer "F.Cu") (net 8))
 (segment (start 142.2875 68.5375) (end 144.6125 68.5375) (width 0.6) (layer "F.Cu") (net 8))
 (segment (start 149.761 91.033902) (end 149.201098 90.474) (width 0.6) (layer "F.Cu") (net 8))
 (segment (start 135.75 88.75) (end 140 88.75) (width 0.6) (layer "F.Cu") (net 8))
 (segment (start 159.964117 99.515996) (end 164.156 95.324112) (width 0.6) (layer "F.Cu") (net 8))
 (segment (start 144.6125 68.5375) (end 151.575 61.575) (width 0.6) (layer "F.Cu") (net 8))
 (segment (start 142.5 89.25) (end 144.75 89.25) (width 0.6) (layer "F.Cu") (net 8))
 (segment (start 142.5 91.533245) (end 150.482754 99.515999) (width 0.6) (layer "F.Cu") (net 8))
 (segment (start 137.628525 66.678525) (end 137.628525 70.835259) (width 0.6) (layer "F.Cu") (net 12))
 (segment (start 134.5 64.15) (end 135.1 64.15) (width 0.6) (layer "F.Cu") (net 12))
 (segment (start 132.35 62) (end 134.5 64.15) (width 0.6) (layer "F.Cu") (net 12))
 (segment (start 123.7 62) (end 123.851 62.151) (width 0.6) (layer "F.Cu") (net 12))
 (segment (start 137.628525 70.835259) (end 140.5 73.706734) (width 0.6) (layer "F.Cu") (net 12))
 (segment (start 124.3 62) (end 132.35 62) (width 0.6) (layer "F.Cu") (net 12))
 (segment (start 140.5 73.706734) (end 140.5 78) (width 0.6) (layer "F.Cu") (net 12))
 (segment (start 135.1 64.15) (end 137.628525 66.678525) (width 0.6) (layer "F.Cu") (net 12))
 (segment (start 123.8 66.5) (end 128.15 66.5) (width 0.6) (layer "F.Cu") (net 10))
 (segment (start 128.15 66.5) (end 132.349 70.699) (width 0.6) (layer "F.Cu") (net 10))
 (segment (start 132.25 70.798) (end 132.25 88.75) (width 0.6) (layer "F.Cu") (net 10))
 (segment (start 132.349 70.699) (end 132.25 70.798) (width 0.6) (layer "F.Cu") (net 10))
 (segment (start 124.2 66.5) (end 127.2 66.5) (width 0.6) (layer "F.Cu") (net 10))
 (segment (start 153.801 72.0135) (end 153.801 76.499) (width 0.6) (layer "F.Cu") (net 15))
 (segment (start 152.7875 71) (end 153.801 72.0135) (width 0.6) (layer "F.Cu") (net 15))
 (segment (start 153.801 76.499) (end 152.5 77.8) (width 0.6) (layer "F.Cu") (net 15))
 (segment (start 151.199 76.301) (end 151.199 78.699) (width 0.6) (layer "F.Cu") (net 6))
 (segment (start 147.365 92.0875) (end 147.365 93.284147) (width 0.6) (layer "F.Cu") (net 6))
 (segment (start 152.5 75) (end 151.199 76.301) (width 0.6) (layer "F.Cu") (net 6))
 (segment (start 159.052017 97.313998) (end 161.954 94.412014) (width 0.6) (layer "F.Cu") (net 6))
 (segment (start 152.16 79.66) (end 157 79.66) (width 0.6) (layer "F.Cu") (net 6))
 (segment (start 161.954 84.614) (end 157 79.66) (width 0.6) (layer "F.Cu") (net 6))
 (segment (start 151.199 78.699) (end 152.16 79.66) (width 0.6) (layer "F.Cu") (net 6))
 (segment (start 161.954 94.412014) (end 161.954 84.614) (width 0.6) (layer "F.Cu") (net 6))
 (segment (start 147.365 93.284147) (end 151.394852 97.313999) (width 0.6) (layer "F.Cu") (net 6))
 (segment (start 151.394852 97.313999) (end 159.052017 97.313998) (width 0.6) (layer "F.Cu") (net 6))
 (segment (start 151.575 64.375) (end 145.7875 70.1625) (width 0.6) (layer "F.Cu") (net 9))
 (segment (start 145.7875 70.1625) (end 145.7875 71.5) (width 0.6) (layer "F.Cu") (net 9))
 (segment (start 146.095 92.0875) (end 146.095 93.571197) (width 0.6) (layer "F.Cu") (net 5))
 (segment (start 163.055 94.868063) (end 163.055 83.175) (width 0.6) (layer "F.Cu") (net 5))
 (segment (start 150.938803 98.414999) (end 159.508067 98.414997) (width 0.6) (layer "F.Cu") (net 5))
 (segment (start 146.095 93.571197) (end 150.938803 98.414999) (width 0.6) (layer "F.Cu") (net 5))
 (segment (start 163.055 83.175) (end 157 77.12) (width 0.6) (layer "F.Cu") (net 5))
 (segment (start 159.508067 98.414997) (end 163.055 94.868063) (width 0.6) (layer "F.Cu") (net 5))
 (segment (start 136 73.5) (end 136 78.554147) (width 0.6) (layer "F.Cu") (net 2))
 (segment (start 149.338902 83.299) (end 155.559 83.299) (width 0.6) (layer "F.Cu") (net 2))
 (segment (start 159.752 93.499916) (end 159.752 87.492) (width 0.6) (layer "F.Cu") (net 2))
 (segment (start 158.139917 95.112) (end 159.752 93.499916) (width 0.6) (layer "F.Cu") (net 2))
 (segment (start 145.452927 88.007074) (end 148.291222 88.007074) (width 0.6) (layer "F.Cu") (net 2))
 (segment (start 148.291222 88.007074) (end 155.396148 95.112) (width 0.6) (layer "F.Cu") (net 2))
 (segment (start 148.635 84.002902) (end 149.338902 83.299) (width 0.6) (layer "F.Cu") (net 2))
 (segment (start 136 78.554147) (end 145.452927 88.007074) (width 0.6) (layer "F.Cu") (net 2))
 (segment (start 155.559 83.299) (end 157 84.74) (width 0.6) (layer "F.Cu") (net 2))
 (segment (start 148.635 84.9125) (end 148.635 84.002902) (width 0.6) (layer "F.Cu") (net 2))
 (segment (start 155.396148 95.112) (end 158.139917 95.112) (width 0.6) (layer "F.Cu") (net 2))
 (segment (start 159.752 87.492) (end 157 84.74) (width 0.6) (layer "F.Cu") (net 2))
 (segment (start 148.635 92.997098) (end 151.850901 96.212999) (width 0.6) (layer "F.Cu") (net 7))
 (segment (start 151.850901 96.212999) (end 158.595967 96.212999) (width 0.6) (layer "F.Cu") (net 7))
 (segment (start 160.853 86.053) (end 157 82.2) (width 0.6) (layer "F.Cu") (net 7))
 (segment (start 158.595967 96.212999) (end 160.853 93.955965) (width 0.6) (layer "F.Cu") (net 7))
 (segment (start 160.853 93.955965) (end 160.853 86.053) (width 0.6) (layer "F.Cu") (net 7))
 (segment (start 148.635 92.0875) (end 148.635 92.997098) (width 0.6) (layer "F.Cu") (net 7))
 (segment (start 154.8125 89.82) (end 157 89.82) (width 0.6) (layer "F.Cu") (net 1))
 (segment (start 149.905 84.9125) (end 154.8125 89.82) (width 0.6) (layer "F.Cu") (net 1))
 (segment (start 148.068902 86.526) (end 149.201098 86.526) (width 0.6) (layer "F.Cu") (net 3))
 (segment (start 147.365 84.9125) (end 147.365 85.822098) (width 0.6) (layer "F.Cu") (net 3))
 (segment (start 145.528902 86.526) (end 146.974 86.526) (width 0.6) (layer "F.Cu") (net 3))
 (segment (start 147.521451 85.978549) (end 148.068902 86.526) (width 0.6) (layer "F.Cu") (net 3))
 (segment (start 142.5 83.497098) (end 145.528902 86.526) (width 0.6) (layer "F.Cu") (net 3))
 (segment (start 158.651 88.931) (end 157 87.28) (width 0.6) (layer "F.Cu") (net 3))
 (segment (start 149.526 86.526) (end 155.349 92.349) (width 0.6) (layer "F.Cu") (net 3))
 (segment (start 157.683867 94.011) (end 158.651 93.043867) (width 0.6) (layer "F.Cu") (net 3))
 (segment (start 155.349 93.043867) (end 156.316133 94.011) (width 0.6) (layer "F.Cu") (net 3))
 (segment (start 147.365 85.822098) (end 147.521451 85.978549) (width 0.6) (layer "F.Cu") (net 3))
 (segment (start 155.349 92.349) (end 155.349 93.043867) (width 0.6) (layer "F.Cu") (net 3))
 (segment (start 149.201098 86.526) (end 149.27 86.457098) (width 0.6) (layer "F.Cu") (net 3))
 (segment (start 158.651 93.043867) (end 158.651 88.931) (width 0.6) (layer "F.Cu") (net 3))
 (segment (start 149.27 86.457098) (end 149.338902 86.526) (width 0.6) (layer "F.Cu") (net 3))
 (segment (start 156.316133 94.011) (end 157.683867 94.011) (width 0.6) (layer "F.Cu") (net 3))
 (segment (start 142.5 78) (end 142.5 83.497098) (width 0.6) (layer "F.Cu") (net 3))
 (segment (start 149.338902 86.526) (end 149.526 86.526) (width 0.6) (layer "F.Cu") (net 3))
 (segment (start 146.974 86.526) (end 147.521451 85.978549) (width 0.6) (layer "F.Cu") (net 3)))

